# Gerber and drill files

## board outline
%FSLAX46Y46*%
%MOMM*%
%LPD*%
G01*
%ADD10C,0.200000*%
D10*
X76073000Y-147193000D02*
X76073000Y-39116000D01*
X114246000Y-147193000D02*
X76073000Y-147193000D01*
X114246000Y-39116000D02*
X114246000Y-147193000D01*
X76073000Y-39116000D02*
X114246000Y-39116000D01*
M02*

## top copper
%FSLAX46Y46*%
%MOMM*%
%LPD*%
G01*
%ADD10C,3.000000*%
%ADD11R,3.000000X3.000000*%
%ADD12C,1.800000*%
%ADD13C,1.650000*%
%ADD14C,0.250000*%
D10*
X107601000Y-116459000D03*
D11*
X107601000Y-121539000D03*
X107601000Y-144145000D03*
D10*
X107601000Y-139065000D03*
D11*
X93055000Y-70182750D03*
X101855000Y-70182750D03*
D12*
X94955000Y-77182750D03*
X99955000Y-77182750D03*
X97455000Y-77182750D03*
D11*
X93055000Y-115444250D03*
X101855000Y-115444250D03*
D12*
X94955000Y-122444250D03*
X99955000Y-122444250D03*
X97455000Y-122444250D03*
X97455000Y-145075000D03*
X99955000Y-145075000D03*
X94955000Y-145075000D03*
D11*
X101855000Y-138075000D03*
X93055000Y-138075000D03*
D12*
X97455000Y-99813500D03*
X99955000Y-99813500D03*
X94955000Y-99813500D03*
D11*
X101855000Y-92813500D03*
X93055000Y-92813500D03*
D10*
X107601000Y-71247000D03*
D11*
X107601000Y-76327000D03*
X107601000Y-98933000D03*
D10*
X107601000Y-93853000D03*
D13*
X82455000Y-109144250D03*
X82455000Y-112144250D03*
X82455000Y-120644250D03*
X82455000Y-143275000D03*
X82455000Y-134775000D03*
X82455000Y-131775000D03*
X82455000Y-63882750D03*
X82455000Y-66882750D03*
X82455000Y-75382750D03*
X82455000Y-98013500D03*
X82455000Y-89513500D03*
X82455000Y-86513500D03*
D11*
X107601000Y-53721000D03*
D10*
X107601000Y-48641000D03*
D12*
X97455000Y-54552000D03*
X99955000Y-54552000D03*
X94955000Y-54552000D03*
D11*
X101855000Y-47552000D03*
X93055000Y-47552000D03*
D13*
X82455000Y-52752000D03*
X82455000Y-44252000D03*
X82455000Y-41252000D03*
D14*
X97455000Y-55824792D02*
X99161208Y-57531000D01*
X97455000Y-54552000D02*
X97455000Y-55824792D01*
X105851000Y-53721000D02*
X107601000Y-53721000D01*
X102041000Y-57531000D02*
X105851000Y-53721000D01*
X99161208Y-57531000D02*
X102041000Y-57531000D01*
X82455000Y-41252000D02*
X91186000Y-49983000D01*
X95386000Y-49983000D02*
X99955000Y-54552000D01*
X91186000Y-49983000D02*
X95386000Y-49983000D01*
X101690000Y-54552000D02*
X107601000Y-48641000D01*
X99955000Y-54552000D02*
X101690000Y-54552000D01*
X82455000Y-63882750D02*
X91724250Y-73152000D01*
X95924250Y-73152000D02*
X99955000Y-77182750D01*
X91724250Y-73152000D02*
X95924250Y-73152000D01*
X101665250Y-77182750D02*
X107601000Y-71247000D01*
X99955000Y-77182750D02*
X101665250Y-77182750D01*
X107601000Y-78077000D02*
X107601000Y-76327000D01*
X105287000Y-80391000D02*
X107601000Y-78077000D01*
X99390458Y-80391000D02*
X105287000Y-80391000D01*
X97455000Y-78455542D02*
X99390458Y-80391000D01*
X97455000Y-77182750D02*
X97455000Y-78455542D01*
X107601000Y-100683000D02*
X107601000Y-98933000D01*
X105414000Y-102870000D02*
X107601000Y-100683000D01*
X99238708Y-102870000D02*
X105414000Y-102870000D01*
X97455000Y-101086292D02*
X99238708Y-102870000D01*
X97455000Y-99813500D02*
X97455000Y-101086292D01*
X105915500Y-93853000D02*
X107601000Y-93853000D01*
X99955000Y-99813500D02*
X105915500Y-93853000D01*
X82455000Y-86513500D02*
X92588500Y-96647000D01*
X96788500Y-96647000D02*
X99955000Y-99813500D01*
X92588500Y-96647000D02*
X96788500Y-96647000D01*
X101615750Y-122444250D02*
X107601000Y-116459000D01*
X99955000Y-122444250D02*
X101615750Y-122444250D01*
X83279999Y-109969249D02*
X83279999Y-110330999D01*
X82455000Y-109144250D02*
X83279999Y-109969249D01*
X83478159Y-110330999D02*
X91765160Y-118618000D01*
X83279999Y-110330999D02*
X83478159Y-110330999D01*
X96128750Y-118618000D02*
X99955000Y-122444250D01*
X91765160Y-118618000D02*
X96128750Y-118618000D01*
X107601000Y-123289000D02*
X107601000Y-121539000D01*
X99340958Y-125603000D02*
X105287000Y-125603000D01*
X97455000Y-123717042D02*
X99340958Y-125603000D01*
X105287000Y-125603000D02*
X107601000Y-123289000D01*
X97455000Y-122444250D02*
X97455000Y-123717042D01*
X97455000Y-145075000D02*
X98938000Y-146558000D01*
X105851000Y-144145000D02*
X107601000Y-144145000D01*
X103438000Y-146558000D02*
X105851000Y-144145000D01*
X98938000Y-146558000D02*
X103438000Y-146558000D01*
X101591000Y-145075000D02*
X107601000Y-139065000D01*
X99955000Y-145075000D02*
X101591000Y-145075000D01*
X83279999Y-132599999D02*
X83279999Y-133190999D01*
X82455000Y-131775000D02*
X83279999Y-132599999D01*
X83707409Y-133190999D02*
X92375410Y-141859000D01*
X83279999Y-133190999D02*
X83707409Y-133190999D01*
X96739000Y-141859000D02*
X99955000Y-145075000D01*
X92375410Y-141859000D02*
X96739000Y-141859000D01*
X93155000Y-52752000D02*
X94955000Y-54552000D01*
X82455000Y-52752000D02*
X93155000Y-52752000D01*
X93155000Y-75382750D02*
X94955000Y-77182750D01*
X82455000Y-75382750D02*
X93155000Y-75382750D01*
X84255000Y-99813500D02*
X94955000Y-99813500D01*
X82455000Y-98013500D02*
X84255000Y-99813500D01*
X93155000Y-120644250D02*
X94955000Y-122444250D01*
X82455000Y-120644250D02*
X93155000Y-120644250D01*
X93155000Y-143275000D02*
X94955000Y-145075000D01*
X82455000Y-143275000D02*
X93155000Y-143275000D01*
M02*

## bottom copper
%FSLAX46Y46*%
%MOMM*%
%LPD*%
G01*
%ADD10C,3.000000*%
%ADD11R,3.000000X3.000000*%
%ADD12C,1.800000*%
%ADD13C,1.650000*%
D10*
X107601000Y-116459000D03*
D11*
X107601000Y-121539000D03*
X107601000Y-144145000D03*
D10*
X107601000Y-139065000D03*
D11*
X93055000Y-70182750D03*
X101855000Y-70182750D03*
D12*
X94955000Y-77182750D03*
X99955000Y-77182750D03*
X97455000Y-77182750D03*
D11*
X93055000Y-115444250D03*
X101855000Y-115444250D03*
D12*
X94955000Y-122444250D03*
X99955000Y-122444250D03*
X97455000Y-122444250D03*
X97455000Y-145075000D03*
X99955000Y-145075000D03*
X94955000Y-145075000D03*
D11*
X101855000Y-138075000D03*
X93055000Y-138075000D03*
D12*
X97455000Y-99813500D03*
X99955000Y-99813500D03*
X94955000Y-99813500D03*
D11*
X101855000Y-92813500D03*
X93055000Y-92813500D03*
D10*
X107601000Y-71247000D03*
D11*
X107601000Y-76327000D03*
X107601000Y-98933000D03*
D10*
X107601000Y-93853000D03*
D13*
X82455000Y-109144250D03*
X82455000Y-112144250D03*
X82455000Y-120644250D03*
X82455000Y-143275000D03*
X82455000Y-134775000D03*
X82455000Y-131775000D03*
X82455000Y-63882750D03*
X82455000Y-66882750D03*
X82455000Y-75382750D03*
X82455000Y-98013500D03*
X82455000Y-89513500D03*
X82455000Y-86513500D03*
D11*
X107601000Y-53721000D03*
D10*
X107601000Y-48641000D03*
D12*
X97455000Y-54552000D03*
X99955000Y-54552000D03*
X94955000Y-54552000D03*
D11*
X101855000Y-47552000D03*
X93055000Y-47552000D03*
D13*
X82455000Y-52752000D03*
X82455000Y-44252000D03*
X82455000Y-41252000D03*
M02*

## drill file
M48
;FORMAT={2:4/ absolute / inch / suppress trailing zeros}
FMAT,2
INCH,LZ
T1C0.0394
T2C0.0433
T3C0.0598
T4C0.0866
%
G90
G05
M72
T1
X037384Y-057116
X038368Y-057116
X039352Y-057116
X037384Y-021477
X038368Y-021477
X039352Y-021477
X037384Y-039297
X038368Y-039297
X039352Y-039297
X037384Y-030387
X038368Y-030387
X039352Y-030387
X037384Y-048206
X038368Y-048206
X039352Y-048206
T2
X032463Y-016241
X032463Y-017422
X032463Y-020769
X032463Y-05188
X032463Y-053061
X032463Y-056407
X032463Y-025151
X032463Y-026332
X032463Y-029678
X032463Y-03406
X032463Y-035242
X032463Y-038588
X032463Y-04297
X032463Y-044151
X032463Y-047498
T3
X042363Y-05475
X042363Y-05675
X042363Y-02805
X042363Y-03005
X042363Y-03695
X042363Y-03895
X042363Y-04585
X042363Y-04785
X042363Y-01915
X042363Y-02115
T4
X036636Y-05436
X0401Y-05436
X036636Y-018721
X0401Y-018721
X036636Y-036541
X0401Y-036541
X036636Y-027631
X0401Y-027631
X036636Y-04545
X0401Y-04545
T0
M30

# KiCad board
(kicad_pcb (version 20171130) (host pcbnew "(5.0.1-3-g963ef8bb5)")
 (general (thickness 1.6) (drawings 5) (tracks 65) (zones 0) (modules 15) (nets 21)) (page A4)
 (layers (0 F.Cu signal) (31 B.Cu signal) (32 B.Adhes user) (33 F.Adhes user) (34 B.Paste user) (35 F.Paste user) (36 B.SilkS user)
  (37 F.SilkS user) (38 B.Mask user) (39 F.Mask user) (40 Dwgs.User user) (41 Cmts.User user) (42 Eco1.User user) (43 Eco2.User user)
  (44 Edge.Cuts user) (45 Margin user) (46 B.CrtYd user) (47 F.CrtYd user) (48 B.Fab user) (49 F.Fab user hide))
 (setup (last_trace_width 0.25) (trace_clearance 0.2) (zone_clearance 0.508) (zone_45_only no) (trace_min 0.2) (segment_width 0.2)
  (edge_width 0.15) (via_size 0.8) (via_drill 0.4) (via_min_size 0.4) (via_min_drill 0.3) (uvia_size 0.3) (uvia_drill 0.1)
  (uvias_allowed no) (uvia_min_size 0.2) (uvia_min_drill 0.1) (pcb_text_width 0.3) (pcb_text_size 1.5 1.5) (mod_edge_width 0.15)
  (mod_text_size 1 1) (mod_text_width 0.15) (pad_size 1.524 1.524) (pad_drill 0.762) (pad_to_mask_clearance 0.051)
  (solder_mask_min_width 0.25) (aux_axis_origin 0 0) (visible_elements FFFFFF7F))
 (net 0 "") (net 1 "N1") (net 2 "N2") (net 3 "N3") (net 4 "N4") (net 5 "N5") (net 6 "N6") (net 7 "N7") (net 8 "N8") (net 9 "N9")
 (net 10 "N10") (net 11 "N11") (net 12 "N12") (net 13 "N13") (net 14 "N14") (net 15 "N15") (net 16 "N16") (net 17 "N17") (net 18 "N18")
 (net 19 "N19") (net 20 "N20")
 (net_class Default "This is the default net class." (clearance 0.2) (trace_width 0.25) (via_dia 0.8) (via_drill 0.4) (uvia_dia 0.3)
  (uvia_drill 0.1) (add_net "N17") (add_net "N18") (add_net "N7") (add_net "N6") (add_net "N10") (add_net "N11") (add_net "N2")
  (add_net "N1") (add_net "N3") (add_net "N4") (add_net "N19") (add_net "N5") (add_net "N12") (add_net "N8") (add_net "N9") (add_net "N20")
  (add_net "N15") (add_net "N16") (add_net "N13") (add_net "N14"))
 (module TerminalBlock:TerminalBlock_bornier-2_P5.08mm (layer F.Cu) (at 107.601 121.539 90)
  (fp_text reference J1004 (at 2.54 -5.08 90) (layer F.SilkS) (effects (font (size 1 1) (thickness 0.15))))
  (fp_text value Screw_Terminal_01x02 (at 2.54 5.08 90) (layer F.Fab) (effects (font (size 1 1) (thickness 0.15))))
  (pad 2 thru_hole circle (at 5.08 0 90) (size 3 3) (drill 1.52) (layers *.Cu *.Mask) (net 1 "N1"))
  (pad 1 thru_hole rect (at 0 0 90) (size 3 3) (drill 1.52) (layers *.Cu *.Mask) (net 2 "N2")))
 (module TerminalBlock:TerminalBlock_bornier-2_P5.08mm (layer F.Cu) (at 107.601 144.145 90)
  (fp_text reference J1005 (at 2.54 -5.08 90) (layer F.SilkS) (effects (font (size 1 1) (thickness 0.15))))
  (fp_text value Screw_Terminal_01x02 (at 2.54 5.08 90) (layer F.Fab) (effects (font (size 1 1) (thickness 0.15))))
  (pad 1 thru_hole rect (at 0 0 90) (size 3 3) (drill 1.52) (layers *.Cu *.Mask) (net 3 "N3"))
  (pad 2 thru_hole circle (at 5.08 0 90) (size 3 3) (drill 1.52) (layers *.Cu *.Mask) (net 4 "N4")))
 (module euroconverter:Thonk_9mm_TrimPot (layer F.Cu) (at 97.455 77.18275)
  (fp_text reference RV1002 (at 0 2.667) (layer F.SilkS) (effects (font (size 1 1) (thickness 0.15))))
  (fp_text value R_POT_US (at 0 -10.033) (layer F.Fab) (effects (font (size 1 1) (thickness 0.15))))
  (pad "" thru_hole rect (at -4.4 -7) (size 3 3) (drill 2.2) (layers *.Cu *.Mask))
  (pad "" thru_hole rect (at 4.4 -7) (size 3 3) (drill 2.2) (layers *.Cu *.Mask))
  (pad 1 thru_hole circle (at -2.5 0) (size 1.8 1.8) (drill 1) (layers *.Cu *.Mask) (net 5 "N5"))
  (pad 3 thru_hole circle (at 2.5 0) (size 1.8 1.8) (drill 1) (layers *.Cu *.Mask) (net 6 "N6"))
  (pad 2 thru_hole circle (at 0 0) (size 1.8 1.8) (drill 1) (layers *.Cu *.Mask) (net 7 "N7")))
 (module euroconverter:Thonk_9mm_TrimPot (layer F.Cu) (at 97.455 122.44425)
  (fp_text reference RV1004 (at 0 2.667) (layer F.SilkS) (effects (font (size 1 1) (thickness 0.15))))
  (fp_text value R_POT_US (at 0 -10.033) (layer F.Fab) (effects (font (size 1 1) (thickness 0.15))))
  (pad "" thru_hole rect (at -4.4 -7) (size 3 3) (drill 2.2) (layers *.Cu *.Mask))
  (pad "" thru_hole rect (at 4.4 -7) (size 3 3) (drill 2.2) (layers *.Cu *.Mask))
  (pad 1 thru_hole circle (at -2.5 0) (size 1.8 1.8) (drill 1) (layers *.Cu *.Mask) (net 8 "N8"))
  (pad 3 thru_hole circle (at 2.5 0) (size 1.8 1.8) (drill 1) (layers *.Cu *.Mask) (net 1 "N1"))
  (pad 2 thru_hole circle (at 0 0) (size 1.8 1.8) (drill 1) (layers *.Cu *.Mask) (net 2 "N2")))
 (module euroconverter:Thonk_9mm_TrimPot (layer F.Cu) (at 97.455 145.075)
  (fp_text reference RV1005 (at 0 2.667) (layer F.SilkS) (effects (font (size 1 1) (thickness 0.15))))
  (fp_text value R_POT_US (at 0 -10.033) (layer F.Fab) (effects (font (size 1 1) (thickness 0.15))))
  (pad 2 thru_hole circle (at 0 0) (size 1.8 1.8) (drill 1) (layers *.Cu *.Mask) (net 3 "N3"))
  (pad 3 thru_hole circle (at 2.5 0) (size 1.8 1.8) (drill 1) (layers *.Cu *.Mask) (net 4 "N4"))
  (pad 1 thru_hole circle (at -2.5 0) (size 1.8 1.8) (drill 1) (layers *.Cu *.Mask) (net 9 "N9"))
  (pad "" thru_hole rect (at 4.4 -7) (size 3 3) (drill 2.2) (layers *.Cu *.Mask))
  (pad "" thru_hole rect (at -4.4 -7) (size 3 3) (drill 2.2) (layers *.Cu *.Mask)))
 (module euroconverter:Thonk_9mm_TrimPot (layer F.Cu) (at 97.455 99.8135)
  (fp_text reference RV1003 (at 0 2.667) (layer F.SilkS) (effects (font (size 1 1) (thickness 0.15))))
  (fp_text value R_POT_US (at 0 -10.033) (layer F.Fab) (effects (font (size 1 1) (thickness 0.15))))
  (pad 2 thru_hole circle (at 0 0) (size 1.8 1.8) (drill 1) (layers *.Cu *.Mask) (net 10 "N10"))
  (pad 3 thru_hole circle (at 2.5 0) (size 1.8 1.8) (drill 1) (layers *.Cu *.Mask) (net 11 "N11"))
  (pad 1 thru_hole circle (at -2.5 0) (size 1.8 1.8) (drill 1) (layers *.Cu *.Mask) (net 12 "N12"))
  (pad "" thru_hole rect (at 4.4 -7) (size 3 3) (drill 2.2) (layers *.Cu *.Mask))
  (pad "" thru_hole rect (at -4.4 -7) (size 3 3) (drill 2.2) (layers *.Cu *.Mask)))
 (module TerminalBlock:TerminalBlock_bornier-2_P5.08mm (layer F.Cu) (at 107.601 76.327 90)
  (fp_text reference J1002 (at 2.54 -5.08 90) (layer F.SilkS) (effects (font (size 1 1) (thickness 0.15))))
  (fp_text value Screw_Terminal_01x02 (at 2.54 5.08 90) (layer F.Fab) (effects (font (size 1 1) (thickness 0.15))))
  (pad 2 thru_hole circle (at 5.08 0 90) (size 3 3) (drill 1.52) (layers *.Cu *.Mask) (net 6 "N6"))
  (pad 1 thru_hole rect (at 0 0 90) (size 3 3) (drill 1.52) (layers *.Cu *.Mask) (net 7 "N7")))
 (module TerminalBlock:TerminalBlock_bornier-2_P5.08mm (layer F.Cu) (at 107.601 98.933 90)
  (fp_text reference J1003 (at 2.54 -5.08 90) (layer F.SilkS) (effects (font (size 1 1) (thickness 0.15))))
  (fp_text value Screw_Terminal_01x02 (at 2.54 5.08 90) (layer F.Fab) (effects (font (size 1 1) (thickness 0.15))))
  (pad 1 thru_hole rect (at 0 0 90) (size 3 3) (drill 1.52) (layers *.Cu *.Mask) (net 10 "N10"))
  (pad 2 thru_hole circle (at 5.08 0 90) (size 3 3) (drill 1.52) (layers *.Cu *.Mask) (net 11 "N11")))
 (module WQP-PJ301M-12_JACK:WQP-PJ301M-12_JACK (layer F.Cu) (at 82.455 115.64425 180)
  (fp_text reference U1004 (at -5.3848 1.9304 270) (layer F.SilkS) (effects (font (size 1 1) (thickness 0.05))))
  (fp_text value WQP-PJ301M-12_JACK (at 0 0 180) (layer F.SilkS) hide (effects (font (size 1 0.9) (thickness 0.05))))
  (pad P$3 thru_hole circle (at 0 6.5 180) (size 1.65 1.65) (drill 1.1) (layers *.Cu *.Mask) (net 1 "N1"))
  (pad P$2 thru_hole circle (at 0 3.5 180) (size 1.65 1.65) (drill 1.1) (layers *.Cu *.Mask) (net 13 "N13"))
  (pad P$1 thru_hole circle (at 0 -5 180) (size 1.65 1.65) (drill 1.1) (layers *.Cu *.Mask) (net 8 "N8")))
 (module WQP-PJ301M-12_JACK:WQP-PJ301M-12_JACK (layer F.Cu) (at 82.455 138.275 180)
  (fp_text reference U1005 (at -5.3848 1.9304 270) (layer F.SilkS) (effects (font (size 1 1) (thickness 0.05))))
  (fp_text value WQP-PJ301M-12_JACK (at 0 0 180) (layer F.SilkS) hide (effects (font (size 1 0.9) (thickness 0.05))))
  (pad P$1 thru_hole circle (at 0 -5 180) (size 1.65 1.65) (drill 1.1) (layers *.Cu *.Mask) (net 9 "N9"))
  (pad P$2 thru_hole circle (at 0 3.5 180) (size 1.65 1.65) (drill 1.1) (layers *.Cu *.Mask) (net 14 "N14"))
  (pad P$3 thru_hole circle (at 0 6.5 180) (size 1.65 1.65) (drill 1.1) (layers *.Cu *.Mask) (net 4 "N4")))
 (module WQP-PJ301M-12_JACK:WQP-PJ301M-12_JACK (layer F.Cu) (at 82.455 70.38275 180)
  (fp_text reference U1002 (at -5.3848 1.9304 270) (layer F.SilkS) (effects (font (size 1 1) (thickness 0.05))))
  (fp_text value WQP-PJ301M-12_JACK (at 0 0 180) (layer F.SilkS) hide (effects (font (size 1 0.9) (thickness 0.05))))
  (pad P$3 thru_hole circle (at 0 6.5 180) (size 1.65 1.65) (drill 1.1) (layers *.Cu *.Mask) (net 6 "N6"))
  (pad P$2 thru_hole circle (at 0 3.5 180) (size 1.65 1.65) (drill 1.1) (layers *.Cu *.Mask) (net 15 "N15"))
  (pad P$1 thru_hole circle (at 0 -5 180) (size 1.65 1.65) (drill 1.1) (layers *.Cu *.Mask) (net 5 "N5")))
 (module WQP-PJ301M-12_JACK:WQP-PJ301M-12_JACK (layer F.Cu) (at 82.455 93.0135 180)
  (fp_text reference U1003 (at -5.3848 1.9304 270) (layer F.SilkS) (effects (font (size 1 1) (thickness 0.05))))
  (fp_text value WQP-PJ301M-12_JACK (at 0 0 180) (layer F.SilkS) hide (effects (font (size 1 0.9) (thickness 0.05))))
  (pad P$1 thru_hole circle (at 0 -5 180) (size 1.65 1.65) (drill 1.1) (layers *.Cu *.Mask) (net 12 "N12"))
  (pad P$2 thru_hole circle (at 0 3.5 180) (size 1.65 1.65) (drill 1.1) (layers *.Cu *.Mask) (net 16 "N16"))
  (pad P$3 thru_hole circle (at 0 6.5 180) (size 1.65 1.65) (drill 1.1) (layers *.Cu *.Mask) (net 11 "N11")))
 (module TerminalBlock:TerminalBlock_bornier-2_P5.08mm (layer F.Cu) (at 107.601 53.721 90)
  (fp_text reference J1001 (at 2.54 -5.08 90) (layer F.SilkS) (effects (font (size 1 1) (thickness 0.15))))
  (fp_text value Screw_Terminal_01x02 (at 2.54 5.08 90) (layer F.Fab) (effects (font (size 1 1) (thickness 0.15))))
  (pad 1 thru_hole rect (at 0 0 90) (size 3 3) (drill 1.52) (layers *.Cu *.Mask) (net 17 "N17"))
  (pad 2 thru_hole circle (at 5.08 0 90) (size 3 3) (drill 1.52) (layers *.Cu *.Mask) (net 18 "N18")))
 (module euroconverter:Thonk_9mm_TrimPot (layer F.Cu) (at 97.455 54.552)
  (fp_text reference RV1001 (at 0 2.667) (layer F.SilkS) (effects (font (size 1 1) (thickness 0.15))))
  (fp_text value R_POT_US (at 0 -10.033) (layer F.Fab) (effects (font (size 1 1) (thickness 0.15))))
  (pad 2 thru_hole circle (at 0 0) (size 1.8 1.8) (drill 1) (layers *.Cu *.Mask) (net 17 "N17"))
  (pad 3 thru_hole circle (at 2.5 0) (size 1.8 1.8) (drill 1) (layers *.Cu *.Mask) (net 18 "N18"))
  (pad 1 thru_hole circle (at -2.5 0) (size 1.8 1.8) (drill 1) (layers *.Cu *.Mask) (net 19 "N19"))
  (pad "" thru_hole rect (at 4.4 -7) (size 3 3) (drill 2.2) (layers *.Cu *.Mask))
  (pad "" thru_hole rect (at -4.4 -7) (size 3 3) (drill 2.2) (layers *.Cu *.Mask)))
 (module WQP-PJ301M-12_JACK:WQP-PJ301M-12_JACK (layer F.Cu) (at 82.455 47.752 180)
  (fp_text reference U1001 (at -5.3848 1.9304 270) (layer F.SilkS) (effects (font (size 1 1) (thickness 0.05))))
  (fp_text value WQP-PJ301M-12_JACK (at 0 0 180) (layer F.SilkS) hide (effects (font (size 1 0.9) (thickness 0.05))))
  (pad P$1 thru_hole circle (at 0 -5 180) (size 1.65 1.65) (drill 1.1) (layers *.Cu *.Mask) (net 19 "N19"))
  (pad P$2 thru_hole circle (at 0 3.5 180) (size 1.65 1.65) (drill 1.1) (layers *.Cu *.Mask) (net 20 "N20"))
  (pad P$3 thru_hole circle (at 0 6.5 180) (size 1.65 1.65) (drill 1.1) (layers *.Cu *.Mask) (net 18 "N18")))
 (gr_line (start 76.073 147.193) (end 76.073 39.116) (layer Edge.Cuts) (width 0.2))
 (gr_line (start 114.246 147.193) (end 76.073 147.193) (layer Edge.Cuts) (width 0.2))
 (gr_line (start 114.246 39.116) (end 114.246 147.193) (layer Edge.Cuts) (width 0.2))
 (gr_line (start 76.073 39.116) (end 114.246 39.116) (layer Edge.Cuts) (width 0.2))
 (segment (start 97.455 55.824792) (end 99.161208 57.531) (width 0.25) (layer F.Cu) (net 17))
 (segment (start 97.455 54.552) (end 97.455 55.824792) (width 0.25) (layer F.Cu) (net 17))
 (segment (start 105.851 53.721) (end 107.601 53.721) (width 0.25) (layer F.Cu) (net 17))
 (segment (start 102.041 57.531) (end 105.851 53.721) (width 0.25) (layer F.Cu) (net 17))
 (segment (start 99.161208 57.531) (end 102.041 57.531) (width 0.25) (layer F.Cu) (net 17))
 (segment (start 82.455 41.252) (end 91.186 49.983) (width 0.25) (layer F.Cu) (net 18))
 (segment (start 95.386 49.983) (end 99.955 54.552) (width 0.25) (layer F.Cu) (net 18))
 (segment (start 91.186 49.983) (end 95.386 49.983) (width 0.25) (layer F.Cu) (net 18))
 (segment (start 101.69 54.552) (end 107.601 48.641) (width 0.25) (layer F.Cu) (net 18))
 (segment (start 99.955 54.552) (end 101.69 54.552) (width 0.25) (layer F.Cu) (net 18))
 (segment (start 82.455 63.88275) (end 91.72425 73.152) (width 0.25) (layer F.Cu) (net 6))
 (segment (start 95.92425 73.152) (end 99.955 77.18275) (width 0.25) (layer F.Cu) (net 6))
 (segment (start 91.72425 73.152) (end 95.92425 73.152) (width 0.25) (layer F.Cu) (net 6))
 (segment (start 101.66525 77.18275) (end 107.601 71.247) (width 0.25) (layer F.Cu) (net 6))
 (segment (start 99.955 77.18275) (end 101.66525 77.18275) (width 0.25) (layer F.Cu) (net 6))
 (segment (start 107.601 78.077) (end 107.601 76.327) (width 0.25) (layer F.Cu) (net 7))
 (segment (start 105.287 80.391) (end 107.601 78.077) (width 0.25) (layer F.Cu) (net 7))
 (segment (start 99.390458 80.391) (end 105.287 80.391) (width 0.25) (layer F.Cu) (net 7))
 (segment (start 97.455 78.455542) (end 99.390458 80.391) (width 0.25) (layer F.Cu) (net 7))
 (segment (start 97.455 77.18275) (end 97.455 78.455542) (width 0.25) (layer F.Cu) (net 7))
 (segment (start 107.601 100.683) (end 107.601 98.933) (width 0.25) (layer F.Cu) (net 10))
 (segment (start 105.414 102.87) (end 107.601 100.683) (width 0.25) (layer F.Cu) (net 10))
 (segment (start 99.238708 102.87) (end 105.414 102.87) (width 0.25) (layer F.Cu) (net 10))
 (segment (start 97.455 101.086292) (end 99.238708 102.87) (width 0.25) (layer F.Cu) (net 10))
 (segment (start 97.455 99.8135) (end 97.455 101.086292) (width 0.25) (layer F.Cu) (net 10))
 (segment (start 105.9155 93.853) (end 107.601 93.853) (width 0.25) (layer F.Cu) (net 11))
 (segment (start 99.955 99.8135) (end 105.9155 93.853) (width 0.25) (layer F.Cu) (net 11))
 (segment (start 82.455 86.5135) (end 92.5885 96.647) (width 0.25) (layer F.Cu) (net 11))
 (segment (start 96.7885 96.647) (end 99.955 99.8135) (width 0.25) (layer F.Cu) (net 11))
 (segment (start 92.5885 96.647) (end 96.7885 96.647) (width 0.25) (layer F.Cu) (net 11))
 (segment (start 101.61575 122.44425) (end 107.601 116.459) (width 0.25) (layer F.Cu) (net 1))
 (segment (start 99.955 122.44425) (end 101.61575 122.44425) (width 0.25) (layer F.Cu) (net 1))
 (segment (start 83.279999 109.969249) (end 83.279999 110.330999) (width 0.25) (layer F.Cu) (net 1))
 (segment (start 82.455 109.14425) (end 83.279999 109.969249) (width 0.25) (layer F.Cu) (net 1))
 (segment (start 83.478159 110.330999) (end 91.76516 118.618) (width 0.25) (layer F.Cu) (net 1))
 (segment (start 83.279999 110.330999) (end 83.478159 110.330999) (width 0.25) (layer F.Cu) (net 1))
 (segment (start 96.12875 118.618) (end 99.955 122.44425) (width 0.25) (layer F.Cu) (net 1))
 (segment (start 91.76516 118.618) (end 96.12875 118.618) (width 0.25) (layer F.Cu) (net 1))
 (segment (start 107.601 123.289) (end 107.601 121.539) (width 0.25) (layer F.Cu) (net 2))
 (segment (start 99.340958 125.603) (end 105.287 125.603) (width 0.25) (layer F.Cu) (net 2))
 (segment (start 97.455 123.717042) (end 99.340958 125.603) (width 0.25) (layer F.Cu) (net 2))
 (segment (start 105.287 125.603) (end 107.601 123.289) (width 0.25) (layer F.Cu) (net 2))
 (segment (start 97.455 122.44425) (end 97.455 123.717042) (width 0.25) (layer F.Cu) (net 2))
 (segment (start 97.455 145.075) (end 98.938 146.558) (width 0.25) (layer F.Cu) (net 3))
 (segment (start 105.851 144.145) (end 107.601 144.145) (width 0.25) (layer F.Cu) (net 3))
 (segment (start 103.438 146.558) (end 105.851 144.145) (width 0.25) (layer F.Cu) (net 3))
 (segment (start 98.938 146.558) (end 103.438 146.558) (width 0.25) (layer F.Cu) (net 3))
 (segment (start 101.591 145.075) (end 107.601 139.065) (width 0.25) (layer F.Cu) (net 4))
 (segment (start 99.955 145.075) (end 101.591 145.075) (width 0.25) (layer F.Cu) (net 4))
 (segment (start 83.279999 132.599999) (end 83.279999 133.190999) (width 0.25) (layer F.Cu) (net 4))
 (segment (start 82.455 131.775) (end 83.279999 132.599999) (width 0.25) (layer F.Cu) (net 4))
 (segment (start 83.707409 133.190999) (end 92.37541 141.859) (width 0.25) (layer F.Cu) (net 4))
 (segment (start 83.279999 133.190999) (end 83.707409 133.190999) (width 0.25) (layer F.Cu) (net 4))
 (segment (start 96.739 141.859) (end 99.955 145.075) (width 0.25) (layer F.Cu) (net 4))
 (segment (start 92.37541 141.859) (end 96.739 141.859) (width 0.25) (layer F.Cu) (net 4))
 (segment (start 93.155 52.752) (end 94.955 54.552) (width 0.25) (layer F.Cu) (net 19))
 (segment (start 82.455 52.752) (end 93.155 52.752) (width 0.25) (layer F.Cu) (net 19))
 (segment (start 93.155 75.38275) (end 94.955 77.18275) (width 0.25) (layer F.Cu) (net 5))
 (segment (start 82.455 75.38275) (end 93.155 75.38275) (width 0.25) (layer F.Cu) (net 5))
 (segment (start 84.255 99.8135) (end 94.955 99.8135) (width 0.25) (layer F.Cu) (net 12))
 (segment (start 82.455 98.0135) (end 84.255 99.8135) (width 0.25) (layer F.Cu) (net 12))
 (segment (start 93.155 120.64425) (end 94.955 122.44425) (width 0.25) (layer F.Cu) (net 8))
 (segment (start 82.455 120.64425) (end 93.155 120.64425) (width 0.25) (layer F.Cu) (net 8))
 (segment (start 93.155 143.275) (end 94.955 145.075) (width 0.25) (layer F.Cu) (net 9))
 (segment (start 82.455 143.275) (end 93.155 143.275) (width 0.25) (layer F.Cu) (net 9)))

